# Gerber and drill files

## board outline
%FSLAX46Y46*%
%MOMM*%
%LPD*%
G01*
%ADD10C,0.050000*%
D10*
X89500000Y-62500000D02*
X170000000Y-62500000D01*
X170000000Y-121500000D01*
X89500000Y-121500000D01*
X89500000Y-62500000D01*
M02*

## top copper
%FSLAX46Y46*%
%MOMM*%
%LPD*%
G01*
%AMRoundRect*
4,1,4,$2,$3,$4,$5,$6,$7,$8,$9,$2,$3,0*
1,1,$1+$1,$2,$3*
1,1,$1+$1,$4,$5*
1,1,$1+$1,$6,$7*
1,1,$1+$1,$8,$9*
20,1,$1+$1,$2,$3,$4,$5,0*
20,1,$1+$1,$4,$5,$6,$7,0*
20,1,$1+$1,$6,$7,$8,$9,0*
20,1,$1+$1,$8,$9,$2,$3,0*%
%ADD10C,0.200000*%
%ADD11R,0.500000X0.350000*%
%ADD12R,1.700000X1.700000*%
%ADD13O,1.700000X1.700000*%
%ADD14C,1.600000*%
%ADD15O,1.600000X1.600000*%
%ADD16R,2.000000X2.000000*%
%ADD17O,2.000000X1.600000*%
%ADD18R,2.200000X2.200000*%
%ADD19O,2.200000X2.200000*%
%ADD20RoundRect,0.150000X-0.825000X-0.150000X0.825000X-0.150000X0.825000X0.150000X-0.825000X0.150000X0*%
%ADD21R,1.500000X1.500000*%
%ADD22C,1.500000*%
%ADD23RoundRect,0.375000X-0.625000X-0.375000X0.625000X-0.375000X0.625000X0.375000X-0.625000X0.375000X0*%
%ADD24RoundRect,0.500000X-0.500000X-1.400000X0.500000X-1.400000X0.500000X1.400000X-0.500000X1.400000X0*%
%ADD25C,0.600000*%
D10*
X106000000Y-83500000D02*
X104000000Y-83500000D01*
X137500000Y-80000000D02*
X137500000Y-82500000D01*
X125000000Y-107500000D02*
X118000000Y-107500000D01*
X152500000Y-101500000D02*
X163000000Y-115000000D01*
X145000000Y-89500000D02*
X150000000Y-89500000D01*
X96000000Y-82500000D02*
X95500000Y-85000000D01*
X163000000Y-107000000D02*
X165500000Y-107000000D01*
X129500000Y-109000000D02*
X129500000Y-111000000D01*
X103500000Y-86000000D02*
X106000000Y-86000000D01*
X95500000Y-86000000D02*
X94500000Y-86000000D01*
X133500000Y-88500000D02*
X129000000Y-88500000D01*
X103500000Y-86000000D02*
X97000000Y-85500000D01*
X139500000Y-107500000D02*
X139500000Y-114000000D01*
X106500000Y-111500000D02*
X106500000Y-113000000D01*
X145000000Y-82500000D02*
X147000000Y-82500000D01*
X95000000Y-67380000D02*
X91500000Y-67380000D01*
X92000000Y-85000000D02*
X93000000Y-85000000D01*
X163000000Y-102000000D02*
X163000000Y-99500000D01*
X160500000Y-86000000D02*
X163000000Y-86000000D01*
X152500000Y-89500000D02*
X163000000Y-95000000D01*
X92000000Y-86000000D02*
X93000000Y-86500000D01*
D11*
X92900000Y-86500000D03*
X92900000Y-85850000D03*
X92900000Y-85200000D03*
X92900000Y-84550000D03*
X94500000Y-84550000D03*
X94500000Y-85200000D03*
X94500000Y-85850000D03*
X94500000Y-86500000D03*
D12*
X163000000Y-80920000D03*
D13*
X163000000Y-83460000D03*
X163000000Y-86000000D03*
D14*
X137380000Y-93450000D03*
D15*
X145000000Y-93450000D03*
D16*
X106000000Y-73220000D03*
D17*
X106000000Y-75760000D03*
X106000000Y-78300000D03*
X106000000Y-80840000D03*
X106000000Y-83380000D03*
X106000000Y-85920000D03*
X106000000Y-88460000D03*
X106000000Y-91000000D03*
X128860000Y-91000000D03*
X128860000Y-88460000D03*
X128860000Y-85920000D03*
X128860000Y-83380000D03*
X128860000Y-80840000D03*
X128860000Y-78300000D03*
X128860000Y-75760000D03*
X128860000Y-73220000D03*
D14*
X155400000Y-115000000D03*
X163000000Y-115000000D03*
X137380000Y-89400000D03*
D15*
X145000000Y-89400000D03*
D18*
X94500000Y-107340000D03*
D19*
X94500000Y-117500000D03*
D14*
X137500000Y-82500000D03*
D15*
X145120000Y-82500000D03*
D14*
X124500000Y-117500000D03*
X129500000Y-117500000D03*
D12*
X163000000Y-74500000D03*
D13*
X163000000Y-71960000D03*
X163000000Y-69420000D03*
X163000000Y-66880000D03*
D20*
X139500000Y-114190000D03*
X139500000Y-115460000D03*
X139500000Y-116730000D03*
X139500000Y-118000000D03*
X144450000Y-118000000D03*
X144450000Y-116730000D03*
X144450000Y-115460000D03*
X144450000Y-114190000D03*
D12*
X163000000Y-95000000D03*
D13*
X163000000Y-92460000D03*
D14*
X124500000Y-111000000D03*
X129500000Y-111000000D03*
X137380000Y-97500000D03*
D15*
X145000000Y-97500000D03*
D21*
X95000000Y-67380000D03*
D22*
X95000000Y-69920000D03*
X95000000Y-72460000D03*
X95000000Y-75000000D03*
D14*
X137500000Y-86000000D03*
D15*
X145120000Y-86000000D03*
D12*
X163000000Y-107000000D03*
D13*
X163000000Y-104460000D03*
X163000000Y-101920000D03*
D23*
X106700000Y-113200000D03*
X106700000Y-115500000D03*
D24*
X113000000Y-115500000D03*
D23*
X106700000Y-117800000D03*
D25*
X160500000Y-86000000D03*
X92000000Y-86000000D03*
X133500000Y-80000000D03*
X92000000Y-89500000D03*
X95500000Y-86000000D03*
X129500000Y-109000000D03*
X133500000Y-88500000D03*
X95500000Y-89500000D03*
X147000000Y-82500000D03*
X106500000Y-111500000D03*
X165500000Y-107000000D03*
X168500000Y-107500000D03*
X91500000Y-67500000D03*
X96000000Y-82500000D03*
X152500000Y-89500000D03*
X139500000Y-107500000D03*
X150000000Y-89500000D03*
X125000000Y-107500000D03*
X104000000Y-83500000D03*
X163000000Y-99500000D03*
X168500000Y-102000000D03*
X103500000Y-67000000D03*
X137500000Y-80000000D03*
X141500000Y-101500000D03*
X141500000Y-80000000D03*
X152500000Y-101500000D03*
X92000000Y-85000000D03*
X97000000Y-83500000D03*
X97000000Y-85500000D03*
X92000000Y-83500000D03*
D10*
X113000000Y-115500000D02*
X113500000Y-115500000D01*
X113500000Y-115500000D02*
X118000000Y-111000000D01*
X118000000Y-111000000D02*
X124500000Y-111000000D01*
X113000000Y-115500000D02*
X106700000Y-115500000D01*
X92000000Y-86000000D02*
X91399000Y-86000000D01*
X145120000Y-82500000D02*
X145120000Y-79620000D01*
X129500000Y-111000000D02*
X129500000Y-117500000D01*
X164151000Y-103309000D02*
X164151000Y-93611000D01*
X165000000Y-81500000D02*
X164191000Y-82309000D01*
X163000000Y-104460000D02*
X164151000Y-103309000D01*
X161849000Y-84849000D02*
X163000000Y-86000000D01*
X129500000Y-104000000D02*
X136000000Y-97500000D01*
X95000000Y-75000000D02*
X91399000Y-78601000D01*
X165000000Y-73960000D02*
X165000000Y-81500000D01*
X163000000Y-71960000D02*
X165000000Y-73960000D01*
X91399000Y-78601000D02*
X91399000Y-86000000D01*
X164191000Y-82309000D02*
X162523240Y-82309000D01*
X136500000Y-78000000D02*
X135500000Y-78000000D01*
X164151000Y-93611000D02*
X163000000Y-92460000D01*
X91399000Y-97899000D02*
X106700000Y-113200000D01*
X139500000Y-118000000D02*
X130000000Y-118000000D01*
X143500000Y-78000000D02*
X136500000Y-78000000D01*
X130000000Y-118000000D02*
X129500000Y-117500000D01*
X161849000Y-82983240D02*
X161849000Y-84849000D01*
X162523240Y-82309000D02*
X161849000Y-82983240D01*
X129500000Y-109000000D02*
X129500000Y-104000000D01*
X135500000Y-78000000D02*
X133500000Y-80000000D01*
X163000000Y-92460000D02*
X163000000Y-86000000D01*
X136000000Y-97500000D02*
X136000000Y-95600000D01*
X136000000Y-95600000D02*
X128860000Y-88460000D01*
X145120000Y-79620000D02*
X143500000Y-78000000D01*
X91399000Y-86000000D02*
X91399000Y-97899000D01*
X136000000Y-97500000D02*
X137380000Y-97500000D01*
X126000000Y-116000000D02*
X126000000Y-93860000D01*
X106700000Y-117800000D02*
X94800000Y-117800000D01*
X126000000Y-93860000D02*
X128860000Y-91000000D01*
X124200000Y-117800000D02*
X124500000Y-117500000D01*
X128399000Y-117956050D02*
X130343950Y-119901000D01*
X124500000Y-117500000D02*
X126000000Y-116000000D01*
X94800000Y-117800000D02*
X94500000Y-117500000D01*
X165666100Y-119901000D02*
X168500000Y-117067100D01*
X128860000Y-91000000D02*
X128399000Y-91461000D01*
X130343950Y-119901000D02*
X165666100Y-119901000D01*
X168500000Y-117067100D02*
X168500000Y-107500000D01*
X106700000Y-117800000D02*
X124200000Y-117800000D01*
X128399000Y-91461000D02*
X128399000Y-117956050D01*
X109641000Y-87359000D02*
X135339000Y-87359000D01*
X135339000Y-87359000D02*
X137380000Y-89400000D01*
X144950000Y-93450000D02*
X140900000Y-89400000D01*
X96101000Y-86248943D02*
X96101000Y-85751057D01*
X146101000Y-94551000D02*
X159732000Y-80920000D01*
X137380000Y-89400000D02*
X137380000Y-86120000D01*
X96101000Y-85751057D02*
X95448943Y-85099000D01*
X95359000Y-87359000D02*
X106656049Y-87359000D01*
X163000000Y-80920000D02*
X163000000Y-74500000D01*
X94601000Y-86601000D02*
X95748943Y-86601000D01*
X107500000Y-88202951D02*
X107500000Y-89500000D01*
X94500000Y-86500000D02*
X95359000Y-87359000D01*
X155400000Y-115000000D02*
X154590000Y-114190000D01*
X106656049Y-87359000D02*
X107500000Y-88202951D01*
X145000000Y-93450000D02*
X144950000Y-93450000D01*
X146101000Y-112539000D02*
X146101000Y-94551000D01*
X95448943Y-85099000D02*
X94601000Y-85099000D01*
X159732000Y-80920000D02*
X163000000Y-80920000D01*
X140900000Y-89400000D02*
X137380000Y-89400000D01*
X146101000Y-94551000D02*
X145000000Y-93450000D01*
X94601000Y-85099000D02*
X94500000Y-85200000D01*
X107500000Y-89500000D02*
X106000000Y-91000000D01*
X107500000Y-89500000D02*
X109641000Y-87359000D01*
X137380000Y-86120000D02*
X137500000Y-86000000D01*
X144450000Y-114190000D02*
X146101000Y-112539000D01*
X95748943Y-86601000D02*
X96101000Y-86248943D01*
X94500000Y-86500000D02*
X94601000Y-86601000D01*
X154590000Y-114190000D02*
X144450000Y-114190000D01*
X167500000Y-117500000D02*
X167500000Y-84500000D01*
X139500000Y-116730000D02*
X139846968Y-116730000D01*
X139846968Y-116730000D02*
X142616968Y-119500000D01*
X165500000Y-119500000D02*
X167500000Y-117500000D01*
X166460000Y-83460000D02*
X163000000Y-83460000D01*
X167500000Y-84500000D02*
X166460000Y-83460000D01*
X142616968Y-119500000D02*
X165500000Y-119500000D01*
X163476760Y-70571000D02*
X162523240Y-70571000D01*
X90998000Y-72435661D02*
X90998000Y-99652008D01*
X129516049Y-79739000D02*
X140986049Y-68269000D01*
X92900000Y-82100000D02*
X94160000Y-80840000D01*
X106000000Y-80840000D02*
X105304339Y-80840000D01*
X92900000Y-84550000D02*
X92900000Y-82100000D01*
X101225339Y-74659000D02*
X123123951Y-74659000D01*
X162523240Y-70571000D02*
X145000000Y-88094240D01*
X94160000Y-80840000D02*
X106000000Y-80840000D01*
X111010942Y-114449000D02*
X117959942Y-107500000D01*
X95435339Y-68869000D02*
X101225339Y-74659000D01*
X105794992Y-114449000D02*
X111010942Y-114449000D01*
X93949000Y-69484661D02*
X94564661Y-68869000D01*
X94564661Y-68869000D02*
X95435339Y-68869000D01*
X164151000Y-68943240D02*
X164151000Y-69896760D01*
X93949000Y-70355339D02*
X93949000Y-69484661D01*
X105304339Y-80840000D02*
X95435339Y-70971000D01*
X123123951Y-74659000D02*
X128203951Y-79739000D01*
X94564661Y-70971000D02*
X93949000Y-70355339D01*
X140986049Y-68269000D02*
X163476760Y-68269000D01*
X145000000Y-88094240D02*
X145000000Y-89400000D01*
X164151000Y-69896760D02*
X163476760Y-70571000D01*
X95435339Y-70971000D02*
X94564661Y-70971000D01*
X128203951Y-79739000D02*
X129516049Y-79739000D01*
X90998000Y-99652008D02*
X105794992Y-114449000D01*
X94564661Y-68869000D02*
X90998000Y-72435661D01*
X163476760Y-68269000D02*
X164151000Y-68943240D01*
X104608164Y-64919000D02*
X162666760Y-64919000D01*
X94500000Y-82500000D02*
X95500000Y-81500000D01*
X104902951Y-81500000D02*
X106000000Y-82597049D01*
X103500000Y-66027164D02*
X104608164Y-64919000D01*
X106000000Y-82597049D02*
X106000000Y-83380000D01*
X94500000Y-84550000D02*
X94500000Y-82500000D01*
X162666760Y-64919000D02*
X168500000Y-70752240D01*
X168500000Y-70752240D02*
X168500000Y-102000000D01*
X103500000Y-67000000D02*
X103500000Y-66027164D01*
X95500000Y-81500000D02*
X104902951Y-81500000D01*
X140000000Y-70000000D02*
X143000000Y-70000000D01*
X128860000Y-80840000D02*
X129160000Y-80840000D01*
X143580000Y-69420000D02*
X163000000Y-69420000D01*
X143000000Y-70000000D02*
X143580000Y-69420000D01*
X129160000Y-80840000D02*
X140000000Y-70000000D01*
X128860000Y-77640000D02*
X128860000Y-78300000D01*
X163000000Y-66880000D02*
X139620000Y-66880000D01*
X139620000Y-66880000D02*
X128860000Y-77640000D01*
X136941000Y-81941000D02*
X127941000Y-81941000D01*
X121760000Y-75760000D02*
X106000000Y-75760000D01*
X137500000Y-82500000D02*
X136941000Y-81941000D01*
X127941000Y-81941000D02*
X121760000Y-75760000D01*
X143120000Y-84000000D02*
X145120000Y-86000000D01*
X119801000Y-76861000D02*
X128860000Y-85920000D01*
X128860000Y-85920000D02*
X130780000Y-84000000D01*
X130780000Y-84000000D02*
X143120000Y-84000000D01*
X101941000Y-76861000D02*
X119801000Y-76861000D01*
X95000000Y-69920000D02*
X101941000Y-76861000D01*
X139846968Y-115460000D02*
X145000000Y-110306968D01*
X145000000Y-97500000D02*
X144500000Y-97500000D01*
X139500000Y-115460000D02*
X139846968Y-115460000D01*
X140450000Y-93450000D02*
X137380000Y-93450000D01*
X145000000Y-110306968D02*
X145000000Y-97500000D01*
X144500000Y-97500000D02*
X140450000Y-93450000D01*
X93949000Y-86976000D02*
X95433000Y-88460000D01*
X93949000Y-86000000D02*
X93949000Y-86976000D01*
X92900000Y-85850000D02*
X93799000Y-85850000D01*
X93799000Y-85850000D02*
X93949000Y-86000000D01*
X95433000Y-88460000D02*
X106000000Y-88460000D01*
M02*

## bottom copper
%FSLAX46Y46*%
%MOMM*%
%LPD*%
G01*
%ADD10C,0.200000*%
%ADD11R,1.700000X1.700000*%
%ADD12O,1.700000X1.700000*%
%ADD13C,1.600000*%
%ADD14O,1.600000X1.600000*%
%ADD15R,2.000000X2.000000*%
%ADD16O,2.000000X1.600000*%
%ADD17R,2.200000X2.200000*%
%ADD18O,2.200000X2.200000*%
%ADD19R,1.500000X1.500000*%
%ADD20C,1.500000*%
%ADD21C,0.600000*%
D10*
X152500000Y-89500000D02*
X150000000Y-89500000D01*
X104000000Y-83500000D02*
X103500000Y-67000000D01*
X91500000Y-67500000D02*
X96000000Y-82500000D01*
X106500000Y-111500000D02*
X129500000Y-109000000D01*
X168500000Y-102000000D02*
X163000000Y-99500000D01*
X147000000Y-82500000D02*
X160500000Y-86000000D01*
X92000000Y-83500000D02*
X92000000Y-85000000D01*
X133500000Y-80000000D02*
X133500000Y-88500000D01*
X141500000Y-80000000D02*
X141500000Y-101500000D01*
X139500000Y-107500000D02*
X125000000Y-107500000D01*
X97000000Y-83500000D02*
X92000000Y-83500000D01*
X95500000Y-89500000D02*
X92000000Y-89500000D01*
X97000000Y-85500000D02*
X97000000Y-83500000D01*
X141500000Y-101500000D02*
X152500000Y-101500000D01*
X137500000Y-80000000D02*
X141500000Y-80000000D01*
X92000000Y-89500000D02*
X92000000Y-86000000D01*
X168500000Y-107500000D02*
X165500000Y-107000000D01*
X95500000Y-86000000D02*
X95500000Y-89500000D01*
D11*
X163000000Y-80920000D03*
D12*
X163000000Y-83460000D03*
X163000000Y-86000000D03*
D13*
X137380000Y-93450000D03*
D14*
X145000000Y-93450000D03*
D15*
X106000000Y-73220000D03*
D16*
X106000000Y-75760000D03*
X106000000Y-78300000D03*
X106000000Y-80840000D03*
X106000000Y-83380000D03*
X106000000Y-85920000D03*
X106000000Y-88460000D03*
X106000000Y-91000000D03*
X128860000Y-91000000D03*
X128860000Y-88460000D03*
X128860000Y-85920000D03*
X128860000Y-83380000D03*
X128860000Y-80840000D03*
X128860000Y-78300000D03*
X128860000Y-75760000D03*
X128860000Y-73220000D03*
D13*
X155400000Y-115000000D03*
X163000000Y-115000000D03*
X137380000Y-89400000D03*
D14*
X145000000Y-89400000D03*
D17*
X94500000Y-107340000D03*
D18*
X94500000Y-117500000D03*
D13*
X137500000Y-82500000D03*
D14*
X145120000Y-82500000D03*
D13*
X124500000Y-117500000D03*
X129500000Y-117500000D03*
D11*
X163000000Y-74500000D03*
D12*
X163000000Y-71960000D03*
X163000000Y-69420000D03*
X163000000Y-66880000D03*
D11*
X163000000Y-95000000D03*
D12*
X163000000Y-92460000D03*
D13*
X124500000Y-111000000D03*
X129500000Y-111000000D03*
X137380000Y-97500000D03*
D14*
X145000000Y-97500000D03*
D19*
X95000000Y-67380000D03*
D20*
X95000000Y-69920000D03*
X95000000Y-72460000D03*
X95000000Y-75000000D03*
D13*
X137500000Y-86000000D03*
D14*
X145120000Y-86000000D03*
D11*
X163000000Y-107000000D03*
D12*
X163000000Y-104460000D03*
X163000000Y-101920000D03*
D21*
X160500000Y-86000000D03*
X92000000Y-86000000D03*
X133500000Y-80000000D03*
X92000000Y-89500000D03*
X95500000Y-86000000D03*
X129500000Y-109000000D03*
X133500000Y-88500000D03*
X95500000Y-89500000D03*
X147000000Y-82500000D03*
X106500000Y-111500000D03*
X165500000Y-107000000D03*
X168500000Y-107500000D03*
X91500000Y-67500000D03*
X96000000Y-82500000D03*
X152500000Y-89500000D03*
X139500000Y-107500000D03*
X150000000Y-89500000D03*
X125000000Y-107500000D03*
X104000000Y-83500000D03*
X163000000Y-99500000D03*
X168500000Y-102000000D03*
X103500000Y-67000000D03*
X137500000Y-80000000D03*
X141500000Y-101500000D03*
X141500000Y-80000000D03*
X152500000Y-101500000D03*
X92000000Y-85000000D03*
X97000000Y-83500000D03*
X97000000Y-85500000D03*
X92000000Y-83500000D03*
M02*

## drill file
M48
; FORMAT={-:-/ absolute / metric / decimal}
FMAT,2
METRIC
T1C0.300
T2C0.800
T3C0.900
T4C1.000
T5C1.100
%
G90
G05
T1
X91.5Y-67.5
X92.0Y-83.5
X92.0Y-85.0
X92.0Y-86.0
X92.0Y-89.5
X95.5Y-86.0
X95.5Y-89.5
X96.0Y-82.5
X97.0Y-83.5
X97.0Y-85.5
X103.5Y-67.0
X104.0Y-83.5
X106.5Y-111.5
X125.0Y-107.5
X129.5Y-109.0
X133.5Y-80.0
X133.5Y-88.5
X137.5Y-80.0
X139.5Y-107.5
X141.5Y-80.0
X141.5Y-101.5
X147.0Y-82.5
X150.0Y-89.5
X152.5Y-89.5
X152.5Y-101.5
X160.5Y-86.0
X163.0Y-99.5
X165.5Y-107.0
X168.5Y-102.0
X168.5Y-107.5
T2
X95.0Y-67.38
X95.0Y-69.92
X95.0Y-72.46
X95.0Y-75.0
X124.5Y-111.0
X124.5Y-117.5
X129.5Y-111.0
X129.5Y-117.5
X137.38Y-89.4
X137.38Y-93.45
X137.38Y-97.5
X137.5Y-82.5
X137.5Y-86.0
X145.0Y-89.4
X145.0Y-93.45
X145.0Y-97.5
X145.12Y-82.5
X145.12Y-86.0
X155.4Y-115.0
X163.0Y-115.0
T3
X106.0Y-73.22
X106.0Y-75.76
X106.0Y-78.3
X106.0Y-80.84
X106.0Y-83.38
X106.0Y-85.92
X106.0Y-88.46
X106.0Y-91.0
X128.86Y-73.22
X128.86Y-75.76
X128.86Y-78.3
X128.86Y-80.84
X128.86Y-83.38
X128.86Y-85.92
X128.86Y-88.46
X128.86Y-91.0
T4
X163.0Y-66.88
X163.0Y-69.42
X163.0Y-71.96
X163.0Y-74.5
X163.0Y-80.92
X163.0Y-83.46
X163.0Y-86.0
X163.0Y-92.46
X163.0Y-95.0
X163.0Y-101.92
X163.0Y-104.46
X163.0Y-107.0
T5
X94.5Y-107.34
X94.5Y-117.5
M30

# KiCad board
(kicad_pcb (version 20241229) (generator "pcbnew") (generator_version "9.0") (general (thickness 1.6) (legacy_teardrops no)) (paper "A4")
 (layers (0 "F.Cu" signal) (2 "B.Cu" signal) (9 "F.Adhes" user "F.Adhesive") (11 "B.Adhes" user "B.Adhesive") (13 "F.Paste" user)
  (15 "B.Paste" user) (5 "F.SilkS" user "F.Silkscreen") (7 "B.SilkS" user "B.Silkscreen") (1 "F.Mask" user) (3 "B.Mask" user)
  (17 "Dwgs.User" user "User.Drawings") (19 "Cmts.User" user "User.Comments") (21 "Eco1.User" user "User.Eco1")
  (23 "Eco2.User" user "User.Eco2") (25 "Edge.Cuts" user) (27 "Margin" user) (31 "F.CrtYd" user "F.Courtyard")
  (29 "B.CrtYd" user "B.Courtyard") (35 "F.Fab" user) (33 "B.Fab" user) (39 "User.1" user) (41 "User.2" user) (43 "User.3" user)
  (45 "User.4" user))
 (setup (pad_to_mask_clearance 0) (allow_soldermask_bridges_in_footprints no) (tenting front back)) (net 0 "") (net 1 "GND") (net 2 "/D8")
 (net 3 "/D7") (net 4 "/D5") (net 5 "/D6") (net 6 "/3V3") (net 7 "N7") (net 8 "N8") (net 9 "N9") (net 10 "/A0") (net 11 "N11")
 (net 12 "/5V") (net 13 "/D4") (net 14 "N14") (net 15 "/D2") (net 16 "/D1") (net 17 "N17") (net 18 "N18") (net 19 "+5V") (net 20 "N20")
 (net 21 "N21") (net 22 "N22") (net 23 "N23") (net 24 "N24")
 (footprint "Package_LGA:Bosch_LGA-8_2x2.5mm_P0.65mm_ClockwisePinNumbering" (layer "F.Cu") (at 93.7 85.525 90)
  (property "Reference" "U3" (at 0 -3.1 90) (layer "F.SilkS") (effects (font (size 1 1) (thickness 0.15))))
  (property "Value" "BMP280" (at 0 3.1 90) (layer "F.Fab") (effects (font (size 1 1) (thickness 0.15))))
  (pad "1" smd rect (at -0.975 -0.8 180) (size 0.5 0.35) (layers "F.Cu" "F.Mask" "F.Paste") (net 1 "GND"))
  (pad "2" smd rect (at -0.325 -0.8 180) (size 0.5 0.35) (layers "F.Cu" "F.Mask" "F.Paste") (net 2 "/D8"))
  (pad "3" smd rect (at 0.325 -0.8 180) (size 0.5 0.35) (layers "F.Cu" "F.Mask" "F.Paste") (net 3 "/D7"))
  (pad "4" smd rect (at 0.975 -0.8 180) (size 0.5 0.35) (layers "F.Cu" "F.Mask" "F.Paste") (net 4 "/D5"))
  (pad "5" smd rect (at 0.975 0.8 180) (size 0.5 0.35) (layers "F.Cu" "F.Mask" "F.Paste") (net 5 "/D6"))
  (pad "6" smd rect (at 0.325 0.8 180) (size 0.5 0.35) (layers "F.Cu" "F.Mask" "F.Paste") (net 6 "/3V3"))
  (pad "7" smd rect (at -0.325 0.8 180) (size 0.5 0.35) (layers "F.Cu" "F.Mask" "F.Paste") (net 1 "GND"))
  (pad "8" smd rect (at -0.975 0.8 180) (size 0.5 0.35) (layers "F.Cu" "F.Mask" "F.Paste") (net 6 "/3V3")))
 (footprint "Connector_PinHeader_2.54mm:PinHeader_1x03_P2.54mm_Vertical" (layer "F.Cu") (at 163 80.92)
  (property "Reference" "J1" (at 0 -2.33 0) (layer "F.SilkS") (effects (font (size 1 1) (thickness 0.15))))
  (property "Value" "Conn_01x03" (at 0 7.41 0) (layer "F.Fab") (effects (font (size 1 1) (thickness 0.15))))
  (pad "1" thru_hole rect (at 0 0) (size 1.7 1.7) (drill 1) (layers "*.Cu" "*.Mask") (remove_unused_layers no) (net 6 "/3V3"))
  (pad "2" thru_hole oval (at 0 2.54) (size 1.7 1.7) (drill 1) (layers "*.Cu" "*.Mask") (remove_unused_layers no) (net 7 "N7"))
  (pad "3" thru_hole oval (at 0 5.08) (size 1.7 1.7) (drill 1) (layers "*.Cu" "*.Mask") (remove_unused_layers no) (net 1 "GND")))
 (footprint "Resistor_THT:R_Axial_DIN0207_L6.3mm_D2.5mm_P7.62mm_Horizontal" (layer "F.Cu") (at 137.38 93.45)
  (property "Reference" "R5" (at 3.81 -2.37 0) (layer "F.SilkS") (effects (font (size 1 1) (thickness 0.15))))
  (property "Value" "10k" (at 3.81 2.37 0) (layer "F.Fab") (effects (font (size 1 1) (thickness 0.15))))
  (pad "1" thru_hole circle (at 0 0) (size 1.6 1.6) (drill 0.8) (layers "*.Cu" "*.Mask") (remove_unused_layers no) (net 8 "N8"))
  (pad "2" thru_hole oval (at 7.62 0) (size 1.6 1.6) (drill 0.8) (layers "*.Cu" "*.Mask") (remove_unused_layers no) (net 6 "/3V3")))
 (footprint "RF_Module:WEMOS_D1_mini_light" (layer "F.Cu") (at 106 73.22)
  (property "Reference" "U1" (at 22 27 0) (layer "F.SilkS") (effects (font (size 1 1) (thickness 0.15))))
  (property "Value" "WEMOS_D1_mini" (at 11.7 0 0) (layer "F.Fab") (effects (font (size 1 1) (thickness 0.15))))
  (pad "1" thru_hole rect (at 0 0) (size 2 2) (drill 0.9) (layers "*.Cu" "*.Mask") (remove_unused_layers no) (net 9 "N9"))
  (pad "2" thru_hole oval (at 0 2.54) (size 2 1.6) (drill 0.9) (layers "*.Cu" "*.Mask") (remove_unused_layers no) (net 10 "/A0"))
  (pad "3" thru_hole oval (at 0 5.08) (size 2 1.6) (drill 0.9) (layers "*.Cu" "*.Mask") (remove_unused_layers no) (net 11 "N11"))
  (pad "4" thru_hole oval (at 0 7.62) (size 2 1.6) (drill 0.9) (layers "*.Cu" "*.Mask") (remove_unused_layers no) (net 4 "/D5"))
  (pad "5" thru_hole oval (at 0 10.16) (size 2 1.6) (drill 0.9) (layers "*.Cu" "*.Mask") (remove_unused_layers no) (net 5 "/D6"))
  (pad "6" thru_hole oval (at 0 12.7) (size 2 1.6) (drill 0.9) (layers "*.Cu" "*.Mask") (remove_unused_layers no) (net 3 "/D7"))
  (pad "7" thru_hole oval (at 0 15.24) (size 2 1.6) (drill 0.9) (layers "*.Cu" "*.Mask") (remove_unused_layers no) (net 2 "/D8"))
  (pad "8" thru_hole oval (at 0 17.78) (size 2 1.6) (drill 0.9) (layers "*.Cu" "*.Mask") (remove_unused_layers no) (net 6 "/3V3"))
  (pad "9" thru_hole oval (at 22.86 17.78) (size 2 1.6) (drill 0.9) (layers "*.Cu" "*.Mask") (remove_unused_layers no) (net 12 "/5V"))
  (pad "10" thru_hole oval (at 22.86 15.24) (size 2 1.6) (drill 0.9) (layers "*.Cu" "*.Mask") (remove_unused_layers no) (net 1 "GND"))
  (pad "11" thru_hole oval (at 22.86 12.7) (size 2 1.6) (drill 0.9) (layers "*.Cu" "*.Mask") (remove_unused_layers no) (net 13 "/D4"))
  (pad "12" thru_hole oval (at 22.86 10.16) (size 2 1.6) (drill 0.9) (layers "*.Cu" "*.Mask") (remove_unused_layers no) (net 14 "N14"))
  (pad "13" thru_hole oval (at 22.86 7.62) (size 2 1.6) (drill 0.9) (layers "*.Cu" "*.Mask") (remove_unused_layers no) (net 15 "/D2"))
  (pad "14" thru_hole oval (at 22.86 5.08) (size 2 1.6) (drill 0.9) (layers "*.Cu" "*.Mask") (remove_unused_layers no) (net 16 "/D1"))
  (pad "15" thru_hole oval (at 22.86 2.54) (size 2 1.6) (drill 0.9) (layers "*.Cu" "*.Mask") (remove_unused_layers no) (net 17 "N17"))
  (pad "16" thru_hole oval (at 22.86 0) (size 2 1.6) (drill 0.9) (layers "*.Cu" "*.Mask") (remove_unused_layers no) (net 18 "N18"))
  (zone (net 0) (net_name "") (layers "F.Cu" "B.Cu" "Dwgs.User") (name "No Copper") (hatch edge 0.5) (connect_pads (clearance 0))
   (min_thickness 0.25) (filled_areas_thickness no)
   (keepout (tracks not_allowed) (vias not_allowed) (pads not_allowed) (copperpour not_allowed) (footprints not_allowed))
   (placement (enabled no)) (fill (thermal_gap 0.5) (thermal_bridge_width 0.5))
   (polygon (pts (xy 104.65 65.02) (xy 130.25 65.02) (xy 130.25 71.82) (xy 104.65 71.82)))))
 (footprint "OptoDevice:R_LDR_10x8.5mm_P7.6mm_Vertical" (layer "F.Cu") (at 155.4 115)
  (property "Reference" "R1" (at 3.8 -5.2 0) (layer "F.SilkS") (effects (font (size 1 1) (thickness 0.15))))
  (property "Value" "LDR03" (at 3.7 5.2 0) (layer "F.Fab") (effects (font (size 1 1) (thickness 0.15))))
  (pad "1" thru_hole circle (at 0 0) (size 1.6 1.6) (drill 0.8) (layers "*.Cu" "*.Mask") (remove_unused_layers no) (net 6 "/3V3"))
  (pad "2" thru_hole circle (at 7.6 0) (size 1.6 1.6) (drill 0.8) (layers "*.Cu" "*.Mask") (remove_unused_layers no) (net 10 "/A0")))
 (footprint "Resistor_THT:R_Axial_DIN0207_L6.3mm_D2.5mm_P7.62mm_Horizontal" (layer "F.Cu") (at 137.38 89.4)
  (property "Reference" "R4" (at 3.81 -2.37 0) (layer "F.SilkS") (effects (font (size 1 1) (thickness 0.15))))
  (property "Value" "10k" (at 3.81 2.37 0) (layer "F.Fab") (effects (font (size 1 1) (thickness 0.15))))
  (pad "1" thru_hole circle (at 0 0) (size 1.6 1.6) (drill 0.8) (layers "*.Cu" "*.Mask") (remove_unused_layers no) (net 6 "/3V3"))
  (pad "2" thru_hole oval (at 7.62 0) (size 1.6 1.6) (drill 0.8) (layers "*.Cu" "*.Mask") (remove_unused_layers no) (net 4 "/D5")))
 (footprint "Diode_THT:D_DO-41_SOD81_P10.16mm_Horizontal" (layer "F.Cu") (at 94.5 107.34 -90)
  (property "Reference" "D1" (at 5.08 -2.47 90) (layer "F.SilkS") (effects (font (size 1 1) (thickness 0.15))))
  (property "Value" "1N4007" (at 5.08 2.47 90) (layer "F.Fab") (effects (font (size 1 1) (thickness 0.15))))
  (pad "1" thru_hole rect (at 0 0 270) (size 2.2 2.2) (drill 1.1) (layers "*.Cu" "*.Mask") (remove_unused_layers no) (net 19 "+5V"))
  (pad "2" thru_hole oval (at 10.16 0 270) (size 2.2 2.2) (drill 1.1) (layers "*.Cu" "*.Mask") (remove_unused_layers no) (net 12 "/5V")))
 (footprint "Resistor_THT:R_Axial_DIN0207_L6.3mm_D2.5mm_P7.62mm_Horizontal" (layer "F.Cu") (at 137.5 82.5)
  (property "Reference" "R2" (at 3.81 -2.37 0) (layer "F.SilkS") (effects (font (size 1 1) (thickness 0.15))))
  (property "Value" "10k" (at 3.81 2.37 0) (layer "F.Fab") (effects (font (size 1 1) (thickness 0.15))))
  (pad "1" thru_hole circle (at 0 0) (size 1.6 1.6) (drill 0.8) (layers "*.Cu" "*.Mask") (remove_unused_layers no) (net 10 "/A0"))
  (pad "2" thru_hole oval (at 7.62 0) (size 1.6 1.6) (drill 0.8) (layers "*.Cu" "*.Mask") (remove_unused_layers no) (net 1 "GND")))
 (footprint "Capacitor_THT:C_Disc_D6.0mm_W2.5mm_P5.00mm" (layer "F.Cu") (at 124.5 117.5)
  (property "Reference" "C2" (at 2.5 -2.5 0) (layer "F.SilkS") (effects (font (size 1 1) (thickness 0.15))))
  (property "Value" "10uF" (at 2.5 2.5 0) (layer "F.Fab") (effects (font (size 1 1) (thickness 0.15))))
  (pad "1" thru_hole circle (at 0 0) (size 1.6 1.6) (drill 0.8) (layers "*.Cu" "*.Mask") (remove_unused_layers no) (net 12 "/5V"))
  (pad "2" thru_hole circle (at 5 0) (size 1.6 1.6) (drill 0.8) (layers "*.Cu" "*.Mask") (remove_unused_layers no) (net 1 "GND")))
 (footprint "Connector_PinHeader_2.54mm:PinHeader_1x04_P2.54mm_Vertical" (layer "F.Cu") (at 163 74.5 180)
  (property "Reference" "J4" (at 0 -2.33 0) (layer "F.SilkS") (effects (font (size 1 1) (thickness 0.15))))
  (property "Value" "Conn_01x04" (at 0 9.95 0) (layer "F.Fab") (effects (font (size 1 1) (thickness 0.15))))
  (pad "1" thru_hole rect (at 0 0 180) (size 1.7 1.7) (drill 1) (layers "*.Cu" "*.Mask") (remove_unused_layers no) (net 6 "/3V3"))
  (pad "2" thru_hole oval (at 0 2.54 180) (size 1.7 1.7) (drill 1) (layers "*.Cu" "*.Mask") (remove_unused_layers no) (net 1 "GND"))
  (pad "3" thru_hole oval (at 0 5.08 180) (size 1.7 1.7) (drill 1) (layers "*.Cu" "*.Mask") (remove_unused_layers no) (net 15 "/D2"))
  (pad "4" thru_hole oval (at 0 7.62 180) (size 1.7 1.7) (drill 1) (layers "*.Cu" "*.Mask") (remove_unused_layers no) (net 16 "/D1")))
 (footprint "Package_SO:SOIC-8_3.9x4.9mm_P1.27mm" (layer "F.Cu") (at 141.975 116.095)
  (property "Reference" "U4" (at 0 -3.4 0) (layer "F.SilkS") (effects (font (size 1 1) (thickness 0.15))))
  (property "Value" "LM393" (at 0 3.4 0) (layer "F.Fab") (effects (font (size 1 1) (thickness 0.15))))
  (pad "1" smd roundrect (at -2.475 -1.905) (size 1.95 0.6) (layers "F.Cu" "F.Mask" "F.Paste") (roundrect_rratio 0.25) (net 4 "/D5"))
  (pad "2" smd roundrect (at -2.475 -0.635) (size 1.95 0.6) (layers "F.Cu" "F.Mask" "F.Paste") (roundrect_rratio 0.25) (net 8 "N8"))
  (pad "3" smd roundrect (at -2.475 0.635) (size 1.95 0.6) (layers "F.Cu" "F.Mask" "F.Paste") (roundrect_rratio 0.25) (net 7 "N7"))
  (pad "4" smd roundrect (at -2.475 1.905) (size 1.95 0.6) (layers "F.Cu" "F.Mask" "F.Paste") (roundrect_rratio 0.25) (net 1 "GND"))
  (pad "5" smd roundrect (at 2.475 1.905) (size 1.95 0.6) (layers "F.Cu" "F.Mask" "F.Paste") (roundrect_rratio 0.25) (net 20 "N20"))
  (pad "6" smd roundrect (at 2.475 0.635) (size 1.95 0.6) (layers "F.Cu" "F.Mask" "F.Paste") (roundrect_rratio 0.25) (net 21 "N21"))
  (pad "7" smd roundrect (at 2.475 -0.635) (size 1.95 0.6) (layers "F.Cu" "F.Mask" "F.Paste") (roundrect_rratio 0.25) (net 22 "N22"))
  (pad "8" smd roundrect (at 2.475 -1.905) (size 1.95 0.6) (layers "F.Cu" "F.Mask" "F.Paste") (roundrect_rratio 0.25) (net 6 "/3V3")))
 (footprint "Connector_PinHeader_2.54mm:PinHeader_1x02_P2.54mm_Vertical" (layer "F.Cu") (at 163 95 180)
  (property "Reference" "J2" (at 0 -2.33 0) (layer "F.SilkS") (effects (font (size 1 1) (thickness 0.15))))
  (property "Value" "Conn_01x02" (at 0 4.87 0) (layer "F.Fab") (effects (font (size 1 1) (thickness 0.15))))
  (pad "1" thru_hole rect (at 0 0 180) (size 1.7 1.7) (drill 1) (layers "*.Cu" "*.Mask") (remove_unused_layers no) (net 4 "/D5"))
  (pad "2" thru_hole oval (at 0 2.54 180) (size 1.7 1.7) (drill 1) (layers "*.Cu" "*.Mask") (remove_unused_layers no) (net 1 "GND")))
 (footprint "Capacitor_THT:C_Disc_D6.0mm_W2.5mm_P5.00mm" (layer "F.Cu") (at 124.5 111)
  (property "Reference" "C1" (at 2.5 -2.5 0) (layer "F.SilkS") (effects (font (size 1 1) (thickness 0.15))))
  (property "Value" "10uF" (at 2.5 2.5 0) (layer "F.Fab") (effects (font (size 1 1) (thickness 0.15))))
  (pad "1" thru_hole circle (at 0 0) (size 1.6 1.6) (drill 0.8) (layers "*.Cu" "*.Mask") (remove_unused_layers no) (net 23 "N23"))
  (pad "2" thru_hole circle (at 5 0) (size 1.6 1.6) (drill 0.8) (layers "*.Cu" "*.Mask") (remove_unused_layers no) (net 1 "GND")))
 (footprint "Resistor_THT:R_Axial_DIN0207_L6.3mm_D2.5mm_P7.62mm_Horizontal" (layer "F.Cu") (at 137.38 97.5)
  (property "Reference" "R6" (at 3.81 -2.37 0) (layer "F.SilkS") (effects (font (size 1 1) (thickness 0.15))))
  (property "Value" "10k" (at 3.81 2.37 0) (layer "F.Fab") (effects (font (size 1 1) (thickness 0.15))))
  (pad "1" thru_hole circle (at 0 0) (size 1.6 1.6) (drill 0.8) (layers "*.Cu" "*.Mask") (remove_unused_layers no) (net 1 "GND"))
  (pad "2" thru_hole oval (at 7.62 0) (size 1.6 1.6) (drill 0.8) (layers "*.Cu" "*.Mask") (remove_unused_layers no) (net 8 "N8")))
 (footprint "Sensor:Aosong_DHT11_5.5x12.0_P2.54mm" (layer "F.Cu") (at 95 67.38)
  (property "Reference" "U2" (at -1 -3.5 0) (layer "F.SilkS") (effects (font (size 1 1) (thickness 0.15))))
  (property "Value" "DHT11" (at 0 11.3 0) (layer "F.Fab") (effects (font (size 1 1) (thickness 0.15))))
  (pad "1" thru_hole rect (at 0 0) (size 1.5 1.5) (drill 0.8) (layers "*.Cu" "*.Mask") (remove_unused_layers no) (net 6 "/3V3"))
  (pad "2" thru_hole circle (at 0 2.54) (size 1.5 1.5) (drill 0.8) (layers "*.Cu" "*.Mask") (remove_unused_layers no) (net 13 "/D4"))
  (pad "3" thru_hole circle (at 0 5.08) (size 1.5 1.5) (drill 0.8) (layers "*.Cu" "*.Mask") (remove_unused_layers no) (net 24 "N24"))
  (pad "4" thru_hole circle (at 0 7.62) (size 1.5 1.5) (drill 0.8) (layers "*.Cu" "*.Mask") (remove_unused_layers no) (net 1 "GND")))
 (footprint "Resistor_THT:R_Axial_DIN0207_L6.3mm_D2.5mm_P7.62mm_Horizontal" (layer "F.Cu") (at 137.5 86)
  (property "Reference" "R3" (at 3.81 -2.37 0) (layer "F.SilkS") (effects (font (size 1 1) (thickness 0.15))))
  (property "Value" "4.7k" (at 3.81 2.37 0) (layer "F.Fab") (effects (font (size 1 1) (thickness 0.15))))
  (pad "1" thru_hole circle (at 0 0) (size 1.6 1.6) (drill 0.8) (layers "*.Cu" "*.Mask") (remove_unused_layers no) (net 6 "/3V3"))
  (pad "2" thru_hole oval (at 7.62 0) (size 1.6 1.6) (drill 0.8) (layers "*.Cu" "*.Mask") (remove_unused_layers no) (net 13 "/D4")))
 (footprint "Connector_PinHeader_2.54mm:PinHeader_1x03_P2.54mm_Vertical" (layer "F.Cu") (at 163 107 180)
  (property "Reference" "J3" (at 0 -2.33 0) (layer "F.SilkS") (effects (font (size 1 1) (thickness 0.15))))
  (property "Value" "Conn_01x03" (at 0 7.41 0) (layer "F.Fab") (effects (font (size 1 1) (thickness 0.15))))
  (pad "1" thru_hole rect (at 0 0 180) (size 1.7 1.7) (drill 1) (layers "*.Cu" "*.Mask") (remove_unused_layers no) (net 12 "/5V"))
  (pad "2" thru_hole oval (at 0 2.54 180) (size 1.7 1.7) (drill 1) (layers "*.Cu" "*.Mask") (remove_unused_layers no) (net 1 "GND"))
  (pad "3" thru_hole oval (at 0 5.08 180) (size 1.7 1.7) (drill 1) (layers "*.Cu" "*.Mask") (remove_unused_layers no) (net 5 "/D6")))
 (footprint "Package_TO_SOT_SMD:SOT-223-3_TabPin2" (layer "F.Cu") (at 109.85 115.5)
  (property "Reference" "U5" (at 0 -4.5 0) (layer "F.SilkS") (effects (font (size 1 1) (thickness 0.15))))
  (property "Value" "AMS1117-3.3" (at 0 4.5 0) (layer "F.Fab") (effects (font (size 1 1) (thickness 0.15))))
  (pad "1" smd roundrect (at -3.15 -2.3) (size 2 1.5) (layers "F.Cu" "F.Mask" "F.Paste") (roundrect_rratio 0.25) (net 1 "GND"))
  (pad "2" smd roundrect (at -3.15 0) (size 2 1.5) (layers "F.Cu" "F.Mask" "F.Paste") (roundrect_rratio 0.25) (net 23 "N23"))
  (pad "2" smd roundrect (at 3.15 0) (size 2 3.8) (layers "F.Cu" "F.Mask" "F.Paste") (roundrect_rratio 0.25) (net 23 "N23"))
  (pad "3" smd roundrect (at -3.15 2.3) (size 2 1.5) (layers "F.Cu" "F.Mask" "F.Paste") (roundrect_rratio 0.25) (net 12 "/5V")))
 (gr_line (start 106 83.5) (end 104 83.5) (stroke (width 0.2) (type default)) (layer "F.Cu") (net 5))
 (gr_line (start 137.5 80) (end 137.5 82.5) (stroke (width 0.2) (type default)) (layer "F.Cu") (net 10))
 (gr_line (start 125 107.5) (end 118 107.5) (stroke (width 0.2) (type default)) (layer "F.Cu") (net 4))
 (gr_line (start 152.5 101.5) (end 163 115) (stroke (width 0.2) (type default)) (layer "F.Cu") (net 10))
 (gr_line (start 145 89.5) (end 150 89.5) (stroke (width 0.2) (type default)) (layer "F.Cu") (net 4))
 (gr_line (start 96 82.5) (end 95.5 85) (stroke (width 0.2) (type default)) (layer "F.Cu") (net 6))
 (gr_line (start 163 107) (end 165.5 107) (stroke (width 0.2) (type default)) (layer "F.Cu") (net 12))
 (gr_line (start 129.5 109) (end 129.5 111) (stroke (width 0.2) (type default)) (layer "F.Cu") (net 1))
 (gr_line (start 103.5 86) (end 106 86) (stroke (width 0.2) (type default)) (layer "F.Cu") (net 3))
 (gr_line (start 95.5 86) (end 94.5 86) (stroke (width 0.2) (type default)) (layer "F.Cu") (net 1))
 (gr_line (start 133.5 88.5) (end 129 88.5) (stroke (width 0.2) (type default)) (layer "F.Cu") (net 1))
 (gr_line (start 103.5 86) (end 97 85.5) (stroke (width 0.2) (type default)) (layer "F.Cu") (net 3))
 (gr_line (start 139.5 107.5) (end 139.5 114) (stroke (width 0.2) (type default)) (layer "F.Cu") (net 4))
 (gr_line (start 106.5 111.5) (end 106.5 113) (stroke (width 0.2) (type default)) (layer "F.Cu") (net 1))
 (gr_line (start 145 82.5) (end 147 82.5) (stroke (width 0.2) (type default)) (layer "F.Cu") (net 1))
 (gr_line (start 95 67.38) (end 91.5 67.38) (stroke (width 0.2) (type default)) (layer "F.Cu") (net 6))
 (gr_line (start 92 85) (end 93 85) (stroke (width 0.2) (type default)) (layer "F.Cu") (net 3))
 (gr_line (start 163 102) (end 163 99.5) (stroke (width 0.2) (type default)) (layer "F.Cu") (net 5))
 (gr_line (start 160.5 86) (end 163 86) (stroke (width 0.2) (type default)) (layer "F.Cu") (net 1))
 (gr_line (start 152.5 89.5) (end 163 95) (stroke (width 0.2) (type default)) (layer "F.Cu") (net 4))
 (gr_line (start 92 86) (end 93 86.5) (stroke (width 0.2) (type default)) (layer "F.Cu") (net 1))
 (gr_line (start 152.5 89.5) (end 150 89.5) (stroke (width 0.2) (type default)) (layer "B.Cu") (net 4))
 (gr_line (start 104 83.5) (end 103.5 67) (stroke (width 0.2) (type default)) (layer "B.Cu") (net 5))
 (gr_line (start 91.5 67.5) (end 96 82.5) (stroke (width 0.2) (type default)) (layer "B.Cu") (net 6))
 (gr_line (start 106.5 111.5) (end 129.5 109) (stroke (width 0.2) (type default)) (layer "B.Cu") (net 1))
 (gr_line (start 168.5 102) (end 163 99.5) (stroke (width 0.2) (type default)) (layer "B.Cu") (net 5))
 (gr_line (start 147 82.5) (end 160.5 86) (stroke (width 0.2) (type default)) (layer "B.Cu") (net 1))
 (gr_line (start 92 83.5) (end 92 85) (stroke (width 0.2) (type default)) (layer "B.Cu") (net 3))
 (gr_line (start 133.5 80) (end 133.5 88.5) (stroke (width 0.2) (type default)) (layer "B.Cu") (net 1))
 (gr_line (start 141.5 80) (end 141.5 101.5) (stroke (width 0.2) (type default)) (layer "B.Cu") (net 10))
 (gr_line (start 139.5 107.5) (end 125 107.5) (stroke (width 0.2) (type default)) (layer "B.Cu") (net 4))
 (gr_line (start 97 83.5) (end 92 83.5) (stroke (width 0.2) (type default)) (layer "B.Cu") (net 3))
 (gr_line (start 95.5 89.5) (end 92 89.5) (stroke (width 0.2) (type default)) (layer "B.Cu") (net 1))
 (gr_line (start 97 85.5) (end 97 83.5) (stroke (width 0.2) (type default)) (layer "B.Cu") (net 3))
 (gr_line (start 141.5 101.5) (end 152.5 101.5) (stroke (width 0.2) (type default)) (layer "B.Cu") (net 10))
 (gr_line (start 137.5 80) (end 141.5 80) (stroke (width 0.2) (type default)) (layer "B.Cu") (net 10))
 (gr_line (start 92 89.5) (end 92 86) (stroke (width 0.2) (type default)) (layer "B.Cu") (net 1))
 (gr_line (start 168.5 107.5) (end 165.5 107) (stroke (width 0.2) (type default)) (layer "B.Cu") (net 12))
 (gr_line (start 95.5 86) (end 95.5 89.5) (stroke (width 0.2) (type default)) (layer "B.Cu") (net 1))
 (gr_rect (start 89.5 62.5) (end 170 121.5) (stroke (width 0.05) (type default)) (fill no) (layer "Edge.Cuts"))
 (segment (start 113 115.5) (end 113.5 115.5) (width 0.2) (layer "F.Cu") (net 23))
 (segment (start 113.5 115.5) (end 118 111) (width 0.2) (layer "F.Cu") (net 23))
 (segment (start 118 111) (end 124.5 111) (width 0.2) (layer "F.Cu") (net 23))
 (segment (start 113 115.5) (end 106.7 115.5) (width 0.2) (layer "F.Cu") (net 23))
 (segment (start 92 86) (end 91.399 86) (width 0.2) (layer "F.Cu") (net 1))
 (segment (start 145.12 82.5) (end 145.12 79.62) (width 0.2) (layer "F.Cu") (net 1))
 (segment (start 129.5 111) (end 129.5 117.5) (width 0.2) (layer "F.Cu") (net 1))
 (segment (start 164.151 103.309) (end 164.151 93.611) (width 0.2) (layer "F.Cu") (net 1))
 (segment (start 165 81.5) (end 164.191 82.309) (width 0.2) (layer "F.Cu") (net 1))
 (segment (start 163 104.46) (end 164.151 103.309) (width 0.2) (layer "F.Cu") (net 1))
 (segment (start 161.849 84.849) (end 163 86) (width 0.2) (layer "F.Cu") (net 1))
 (segment (start 129.5 104) (end 136 97.5) (width 0.2) (layer "F.Cu") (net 1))
 (segment (start 95 75) (end 91.399 78.601) (width 0.2) (layer "F.Cu") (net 1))
 (segment (start 165 73.96) (end 165 81.5) (width 0.2) (layer "F.Cu") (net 1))
 (segment (start 163 71.96) (end 165 73.96) (width 0.2) (layer "F.Cu") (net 1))
 (segment (start 91.399 78.601) (end 91.399 86) (width 0.2) (layer "F.Cu") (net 1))
 (segment (start 164.191 82.309) (end 162.52324 82.309) (width 0.2) (layer "F.Cu") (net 1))
 (segment (start 136.5 78) (end 135.5 78) (width 0.2) (layer "F.Cu") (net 1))
 (segment (start 164.151 93.611) (end 163 92.46) (width 0.2) (layer "F.Cu") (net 1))
 (segment (start 91.399 97.899) (end 106.7 113.2) (width 0.2) (layer "F.Cu") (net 1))
 (segment (start 139.5 118) (end 130 118) (width 0.2) (layer "F.Cu") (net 1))
 (segment (start 143.5 78) (end 136.5 78) (width 0.2) (layer "F.Cu") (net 1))
 (segment (start 130 118) (end 129.5 117.5) (width 0.2) (layer "F.Cu") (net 1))
 (segment (start 161.849 82.98324) (end 161.849 84.849) (width 0.2) (layer "F.Cu") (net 1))
 (segment (start 162.52324 82.309) (end 161.849 82.98324) (width 0.2) (layer "F.Cu") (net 1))
 (segment (start 129.5 109) (end 129.5 104) (width 0.2) (layer "F.Cu") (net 1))
 (segment (start 135.5 78) (end 133.5 80) (width 0.2) (layer "F.Cu") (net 1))
 (segment (start 163 92.46) (end 163 86) (width 0.2) (layer "F.Cu") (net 1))
 (segment (start 136 97.5) (end 136 95.6) (width 0.2) (layer "F.Cu") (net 1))
 (segment (start 136 95.6) (end 128.86 88.46) (width 0.2) (layer "F.Cu") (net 1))
 (segment (start 145.12 79.62) (end 143.5 78) (width 0.2) (layer "F.Cu") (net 1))
 (segment (start 91.399 86) (end 91.399 97.899) (width 0.2) (layer "F.Cu") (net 1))
 (segment (start 136 97.5) (end 137.38 97.5) (width 0.2) (layer "F.Cu") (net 1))
 (via (at 160.5 86) (size 0.6) (drill 0.3) (layers "F.Cu" "B.Cu") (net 1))
 (via (at 92 86) (size 0.6) (drill 0.3) (layers "F.Cu" "B.Cu") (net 1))
 (via (at 133.5 80) (size 0.6) (drill 0.3) (layers "F.Cu" "B.Cu") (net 1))
 (via (at 92 89.5) (size 0.6) (drill 0.3) (layers "F.Cu" "B.Cu") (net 1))
 (via (at 95.5 86) (size 0.6) (drill 0.3) (layers "F.Cu" "B.Cu") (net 1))
 (via (at 129.5 109) (size 0.6) (drill 0.3) (layers "F.Cu" "B.Cu") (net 1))
 (via (at 133.5 88.5) (size 0.6) (drill 0.3) (layers "F.Cu" "B.Cu") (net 1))
 (via (at 95.5 89.5) (size 0.6) (drill 0.3) (layers "F.Cu" "B.Cu") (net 1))
 (via (at 147 82.5) (size 0.6) (drill 0.3) (layers "F.Cu" "B.Cu") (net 1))
 (via (at 106.5 111.5) (size 0.6) (drill 0.3) (layers "F.Cu" "B.Cu") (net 1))
 (segment (start 126 116) (end 126 93.86) (width 0.2) (layer "F.Cu") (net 12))
 (segment (start 106.7 117.8) (end 94.8 117.8) (width 0.2) (layer "F.Cu") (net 12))
 (segment (start 126 93.86) (end 128.86 91) (width 0.2) (layer "F.Cu") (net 12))
 (segment (start 124.2 117.8) (end 124.5 117.5) (width 0.2) (layer "F.Cu") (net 12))
 (segment (start 128.399 117.95605) (end 130.34395 119.901) (width 0.2) (layer "F.Cu") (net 12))
 (segment (start 124.5 117.5) (end 126 116) (width 0.2) (layer "F.Cu") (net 12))
 (segment (start 94.8 117.8) (end 94.5 117.5) (width 0.2) (layer "F.Cu") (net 12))
 (segment (start 165.6661 119.901) (end 168.5 117.0671) (width 0.2) (layer "F.Cu") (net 12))
 (segment (start 128.86 91) (end 128.399 91.461) (width 0.2) (layer "F.Cu") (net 12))
 (segment (start 130.34395 119.901) (end 165.6661 119.901) (width 0.2) (layer "F.Cu") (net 12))
 (segment (start 168.5 117.0671) (end 168.5 107.5) (width 0.2) (layer "F.Cu") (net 12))
 (segment (start 106.7 117.8) (end 124.2 117.8) (width 0.2) (layer "F.Cu") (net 12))
 (segment (start 128.399 91.461) (end 128.399 117.95605) (width 0.2) (layer "F.Cu") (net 12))
 (via (at 165.5 107) (size 0.6) (drill 0.3) (layers "F.Cu" "B.Cu") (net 12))
 (via (at 168.5 107.5) (size 0.6) (drill 0.3) (layers "F.Cu" "B.Cu") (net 12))
 (segment (start 109.641 87.359) (end 135.339 87.359) (width 0.2) (layer "F.Cu") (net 6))
 (segment (start 135.339 87.359) (end 137.38 89.4) (width 0.2) (layer "F.Cu") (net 6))
 (segment (start 144.95 93.45) (end 140.9 89.4) (width 0.2) (layer "F.Cu") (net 6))
 (segment (start 96.101 86.248943) (end 96.101 85.751057) (width 0.2) (layer "F.Cu") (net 6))
 (segment (start 146.101 94.551) (end 159.732 80.92) (width 0.2) (layer "F.Cu") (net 6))
 (segment (start 137.38 89.4) (end 137.38 86.12) (width 0.2) (layer "F.Cu") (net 6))
 (segment (start 96.101 85.751057) (end 95.448943 85.099) (width 0.2) (layer "F.Cu") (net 6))
 (segment (start 95.359 87.359) (end 106.656049 87.359) (width 0.2) (layer "F.Cu") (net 6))
 (segment (start 163 80.92) (end 163 74.5) (width 0.2) (layer "F.Cu") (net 6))
 (segment (start 94.601 86.601) (end 95.748943 86.601) (width 0.2) (layer "F.Cu") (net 6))
 (segment (start 107.5 88.202951) (end 107.5 89.5) (width 0.2) (layer "F.Cu") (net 6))
 (segment (start 94.5 86.5) (end 95.359 87.359) (width 0.2) (layer "F.Cu") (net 6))
 (segment (start 155.4 115) (end 154.59 114.19) (width 0.2) (layer "F.Cu") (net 6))
 (segment (start 106.656049 87.359) (end 107.5 88.202951) (width 0.2) (layer "F.Cu") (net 6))
 (segment (start 145 93.45) (end 144.95 93.45) (width 0.2) (layer "F.Cu") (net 6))
 (segment (start 146.101 112.539) (end 146.101 94.551) (width 0.2) (layer "F.Cu") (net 6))
 (segment (start 95.448943 85.099) (end 94.601 85.099) (width 0.2) (layer "F.Cu") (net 6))
 (segment (start 159.732 80.92) (end 163 80.92) (width 0.2) (layer "F.Cu") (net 6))
 (segment (start 140.9 89.4) (end 137.38 89.4) (width 0.2) (layer "F.Cu") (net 6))
 (segment (start 146.101 94.551) (end 145 93.45) (width 0.2) (layer "F.Cu") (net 6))
 (segment (start 94.601 85.099) (end 94.5 85.2) (width 0.2) (layer "F.Cu") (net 6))
 (segment (start 107.5 89.5) (end 106 91) (width 0.2) (layer "F.Cu") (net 6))
 (segment (start 107.5 89.5) (end 109.641 87.359) (width 0.2) (layer "F.Cu") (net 6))
 (segment (start 137.38 86.12) (end 137.5 86) (width 0.2) (layer "F.Cu") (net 6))
 (segment (start 144.45 114.19) (end 146.101 112.539) (width 0.2) (layer "F.Cu") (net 6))
 (segment (start 95.748943 86.601) (end 96.101 86.248943) (width 0.2) (layer "F.Cu") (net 6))
 (segment (start 94.5 86.5) (end 94.601 86.601) (width 0.2) (layer "F.Cu") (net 6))
 (segment (start 154.59 114.19) (end 144.45 114.19) (width 0.2) (layer "F.Cu") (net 6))
 (via (at 91.5 67.5) (size 0.6) (drill 0.3) (layers "F.Cu" "B.Cu") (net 6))
 (via (at 96 82.5) (size 0.6) (drill 0.3) (layers "F.Cu" "B.Cu") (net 6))
 (segment (start 167.5 117.5) (end 167.5 84.5) (width 0.2) (layer "F.Cu") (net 7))
 (segment (start 139.5 116.73) (end 139.846968 116.73) (width 0.2) (layer "F.Cu") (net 7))
 (segment (start 139.846968 116.73) (end 142.616968 119.5) (width 0.2) (layer "F.Cu") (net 7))
 (segment (start 165.5 119.5) (end 167.5 117.5) (width 0.2) (layer "F.Cu") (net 7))
 (segment (start 166.46 83.46) (end 163 83.46) (width 0.2) (layer "F.Cu") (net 7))
 (segment (start 167.5 84.5) (end 166.46 83.46) (width 0.2) (layer "F.Cu") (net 7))
 (segment (start 142.616968 119.5) (end 165.5 119.5) (width 0.2) (layer "F.Cu") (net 7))
 (segment (start 163.47676 70.571) (end 162.52324 70.571) (width 0.2) (layer "F.Cu") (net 4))
 (segment (start 90.998 72.435661) (end 90.998 99.652008) (width 0.2) (layer "F.Cu") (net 4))
 (segment (start 129.516049 79.739) (end 140.986049 68.269) (width 0.2) (layer "F.Cu") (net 4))
 (segment (start 92.9 82.1) (end 94.16 80.84) (width 0.2) (layer "F.Cu") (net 4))
 (segment (start 106 80.84) (end 105.304339 80.84) (width 0.2) (layer "F.Cu") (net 4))
 (segment (start 92.9 84.55) (end 92.9 82.1) (width 0.2) (layer "F.Cu") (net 4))
 (segment (start 101.225339 74.659) (end 123.123951 74.659) (width 0.2) (layer "F.Cu") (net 4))
 (segment (start 162.52324 70.571) (end 145 88.09424) (width 0.2) (layer "F.Cu") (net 4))
 (segment (start 94.16 80.84) (end 106 80.84) (width 0.2) (layer "F.Cu") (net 4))
 (segment (start 111.010942 114.449) (end 117.959942 107.5) (width 0.2) (layer "F.Cu") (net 4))
 (segment (start 95.435339 68.869) (end 101.225339 74.659) (width 0.2) (layer "F.Cu") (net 4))
 (segment (start 105.794992 114.449) (end 111.010942 114.449) (width 0.2) (layer "F.Cu") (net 4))
 (segment (start 93.949 69.484661) (end 94.564661 68.869) (width 0.2) (layer "F.Cu") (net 4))
 (segment (start 94.564661 68.869) (end 95.435339 68.869) (width 0.2) (layer "F.Cu") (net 4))
 (segment (start 164.151 68.94324) (end 164.151 69.89676) (width 0.2) (layer "F.Cu") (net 4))
 (segment (start 93.949 70.355339) (end 93.949 69.484661) (width 0.2) (layer "F.Cu") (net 4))
 (segment (start 105.304339 80.84) (end 95.435339 70.971) (width 0.2) (layer "F.Cu") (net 4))
 (segment (start 123.123951 74.659) (end 128.203951 79.739) (width 0.2) (layer "F.Cu") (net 4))
 (segment (start 94.564661 70.971) (end 93.949 70.355339) (width 0.2) (layer "F.Cu") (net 4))
 (segment (start 140.986049 68.269) (end 163.47676 68.269) (width 0.2) (layer "F.Cu") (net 4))
 (segment (start 145 88.09424) (end 145 89.4) (width 0.2) (layer "F.Cu") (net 4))
 (segment (start 164.151 69.89676) (end 163.47676 70.571) (width 0.2) (layer "F.Cu") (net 4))
 (segment (start 95.435339 70.971) (end 94.564661 70.971) (width 0.2) (layer "F.Cu") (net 4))
 (segment (start 128.203951 79.739) (end 129.516049 79.739) (width 0.2) (layer "F.Cu") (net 4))
 (segment (start 90.998 99.652008) (end 105.794992 114.449) (width 0.2) (layer "F.Cu") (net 4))
 (segment (start 94.564661 68.869) (end 90.998 72.435661) (width 0.2) (layer "F.Cu") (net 4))
 (segment (start 163.47676 68.269) (end 164.151 68.94324) (width 0.2) (layer "F.Cu") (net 4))
 (via (at 152.5 89.5) (size 0.6) (drill 0.3) (layers "F.Cu" "B.Cu") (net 4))
 (via (at 139.5 107.5) (size 0.6) (drill 0.3) (layers "F.Cu" "B.Cu") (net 4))
 (via (at 150 89.5) (size 0.6) (drill 0.3) (layers "F.Cu" "B.Cu") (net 4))
 (via (at 125 107.5) (size 0.6) (drill 0.3) (layers "F.Cu" "B.Cu") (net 4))
 (segment (start 104.608164 64.919) (end 162.66676 64.919) (width 0.2) (layer "F.Cu") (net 5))
 (segment (start 94.5 82.5) (end 95.5 81.5) (width 0.2) (layer "F.Cu") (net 5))
 (segment (start 104.902951 81.5) (end 106 82.597049) (width 0.2) (layer "F.Cu") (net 5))
 (segment (start 103.5 66.027164) (end 104.608164 64.919) (width 0.2) (layer "F.Cu") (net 5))
 (segment (start 106 82.597049) (end 106 83.38) (width 0.2) (layer "F.Cu") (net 5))
 (segment (start 94.5 84.55) (end 94.5 82.5) (width 0.2) (layer "F.Cu") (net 5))
 (segment (start 162.66676 64.919) (end 168.5 70.75224) (width 0.2) (layer "F.Cu") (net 5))
 (segment (start 168.5 70.75224) (end 168.5 102) (width 0.2) (layer "F.Cu") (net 5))
 (segment (start 103.5 67) (end 103.5 66.027164) (width 0.2) (layer "F.Cu") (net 5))
 (segment (start 95.5 81.5) (end 104.902951 81.5) (width 0.2) (layer "F.Cu") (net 5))
 (via (at 104 83.5) (size 0.6) (drill 0.3) (layers "F.Cu" "B.Cu") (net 5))
 (via (at 163 99.5) (size 0.6) (drill 0.3) (layers "F.Cu" "B.Cu") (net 5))
 (via (at 168.5 102) (size 0.6) (drill 0.3) (layers "F.Cu" "B.Cu") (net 5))
 (via (at 103.5 67) (size 0.6) (drill 0.3) (layers "F.Cu" "B.Cu") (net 5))
 (segment (start 140 70) (end 143 70) (width 0.2) (layer "F.Cu") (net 15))
 (segment (start 128.86 80.84) (end 129.16 80.84) (width 0.2) (layer "F.Cu") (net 15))
 (segment (start 143.58 69.42) (end 163 69.42) (width 0.2) (layer "F.Cu") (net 15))
 (segment (start 143 70) (end 143.58 69.42) (width 0.2) (layer "F.Cu") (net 15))
 (segment (start 129.16 80.84) (end 140 70) (width 0.2) (layer "F.Cu") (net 15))
 (segment (start 128.86 77.64) (end 128.86 78.3) (width 0.2) (layer "F.Cu") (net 16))
 (segment (start 163 66.88) (end 139.62 66.88) (width 0.2) (layer "F.Cu") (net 16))
 (segment (start 139.62 66.88) (end 128.86 77.64) (width 0.2) (layer "F.Cu") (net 16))
 (segment (start 136.941 81.941) (end 127.941 81.941) (width 0.2) (layer "F.Cu") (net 10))
 (segment (start 121.76 75.76) (end 106 75.76) (width 0.2) (layer "F.Cu") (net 10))
 (segment (start 137.5 82.5) (end 136.941 81.941) (width 0.2) (layer "F.Cu") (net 10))
 (segment (start 127.941 81.941) (end 121.76 75.76) (width 0.2) (layer "F.Cu") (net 10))
 (via (at 137.5 80) (size 0.6) (drill 0.3) (layers "F.Cu" "B.Cu") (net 10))
 (via (at 141.5 101.5) (size 0.6) (drill 0.3) (layers "F.Cu" "B.Cu") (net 10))
 (via (at 141.5 80) (size 0.6) (drill 0.3) (layers "F.Cu" "B.Cu") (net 10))
 (via (at 152.5 101.5) (size 0.6) (drill 0.3) (layers "F.Cu" "B.Cu") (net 10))
 (segment (start 143.12 84) (end 145.12 86) (width 0.2) (layer "F.Cu") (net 13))
 (segment (start 119.801 76.861) (end 128.86 85.92) (width 0.2) (layer "F.Cu") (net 13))
 (segment (start 128.86 85.92) (end 130.78 84) (width 0.2) (layer "F.Cu") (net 13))
 (segment (start 130.78 84) (end 143.12 84) (width 0.2) (layer "F.Cu") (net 13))
 (segment (start 101.941 76.861) (end 119.801 76.861) (width 0.2) (layer "F.Cu") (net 13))
 (segment (start 95 69.92) (end 101.941 76.861) (width 0.2) (layer "F.Cu") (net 13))
 (segment (start 139.846968 115.46) (end 145 110.306968) (width 0.2) (layer "F.Cu") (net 8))
 (segment (start 145 97.5) (end 144.5 97.5) (width 0.2) (layer "F.Cu") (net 8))
 (segment (start 139.5 115.46) (end 139.846968 115.46) (width 0.2) (layer "F.Cu") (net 8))
 (segment (start 140.45 93.45) (end 137.38 93.45) (width 0.2) (layer "F.Cu") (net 8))
 (segment (start 145 110.306968) (end 145 97.5) (width 0.2) (layer "F.Cu") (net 8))
 (segment (start 144.5 97.5) (end 140.45 93.45) (width 0.2) (layer "F.Cu") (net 8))
 (segment (start 93.949 86.976) (end 95.433 88.46) (width 0.2) (layer "F.Cu") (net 2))
 (segment (start 93.949 86) (end 93.949 86.976) (width 0.2) (layer "F.Cu") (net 2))
 (segment (start 92.9 85.85) (end 93.799 85.85) (width 0.2) (layer "F.Cu") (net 2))
 (segment (start 93.799 85.85) (end 93.949 86) (width 0.2) (layer "F.Cu") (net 2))
 (segment (start 95.433 88.46) (end 106 88.46) (width 0.2) (layer "F.Cu") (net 2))
 (via (at 92 85) (size 0.6) (drill 0.3) (layers "F.Cu" "B.Cu") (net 3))
 (via (at 97 83.5) (size 0.6) (drill 0.3) (layers "F.Cu" "B.Cu") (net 3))
 (via (at 97 85.5) (size 0.6) (drill 0.3) (layers "F.Cu" "B.Cu") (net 3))
 (via (at 92 83.5) (size 0.6) (drill 0.3) (layers "F.Cu" "B.Cu") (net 3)))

